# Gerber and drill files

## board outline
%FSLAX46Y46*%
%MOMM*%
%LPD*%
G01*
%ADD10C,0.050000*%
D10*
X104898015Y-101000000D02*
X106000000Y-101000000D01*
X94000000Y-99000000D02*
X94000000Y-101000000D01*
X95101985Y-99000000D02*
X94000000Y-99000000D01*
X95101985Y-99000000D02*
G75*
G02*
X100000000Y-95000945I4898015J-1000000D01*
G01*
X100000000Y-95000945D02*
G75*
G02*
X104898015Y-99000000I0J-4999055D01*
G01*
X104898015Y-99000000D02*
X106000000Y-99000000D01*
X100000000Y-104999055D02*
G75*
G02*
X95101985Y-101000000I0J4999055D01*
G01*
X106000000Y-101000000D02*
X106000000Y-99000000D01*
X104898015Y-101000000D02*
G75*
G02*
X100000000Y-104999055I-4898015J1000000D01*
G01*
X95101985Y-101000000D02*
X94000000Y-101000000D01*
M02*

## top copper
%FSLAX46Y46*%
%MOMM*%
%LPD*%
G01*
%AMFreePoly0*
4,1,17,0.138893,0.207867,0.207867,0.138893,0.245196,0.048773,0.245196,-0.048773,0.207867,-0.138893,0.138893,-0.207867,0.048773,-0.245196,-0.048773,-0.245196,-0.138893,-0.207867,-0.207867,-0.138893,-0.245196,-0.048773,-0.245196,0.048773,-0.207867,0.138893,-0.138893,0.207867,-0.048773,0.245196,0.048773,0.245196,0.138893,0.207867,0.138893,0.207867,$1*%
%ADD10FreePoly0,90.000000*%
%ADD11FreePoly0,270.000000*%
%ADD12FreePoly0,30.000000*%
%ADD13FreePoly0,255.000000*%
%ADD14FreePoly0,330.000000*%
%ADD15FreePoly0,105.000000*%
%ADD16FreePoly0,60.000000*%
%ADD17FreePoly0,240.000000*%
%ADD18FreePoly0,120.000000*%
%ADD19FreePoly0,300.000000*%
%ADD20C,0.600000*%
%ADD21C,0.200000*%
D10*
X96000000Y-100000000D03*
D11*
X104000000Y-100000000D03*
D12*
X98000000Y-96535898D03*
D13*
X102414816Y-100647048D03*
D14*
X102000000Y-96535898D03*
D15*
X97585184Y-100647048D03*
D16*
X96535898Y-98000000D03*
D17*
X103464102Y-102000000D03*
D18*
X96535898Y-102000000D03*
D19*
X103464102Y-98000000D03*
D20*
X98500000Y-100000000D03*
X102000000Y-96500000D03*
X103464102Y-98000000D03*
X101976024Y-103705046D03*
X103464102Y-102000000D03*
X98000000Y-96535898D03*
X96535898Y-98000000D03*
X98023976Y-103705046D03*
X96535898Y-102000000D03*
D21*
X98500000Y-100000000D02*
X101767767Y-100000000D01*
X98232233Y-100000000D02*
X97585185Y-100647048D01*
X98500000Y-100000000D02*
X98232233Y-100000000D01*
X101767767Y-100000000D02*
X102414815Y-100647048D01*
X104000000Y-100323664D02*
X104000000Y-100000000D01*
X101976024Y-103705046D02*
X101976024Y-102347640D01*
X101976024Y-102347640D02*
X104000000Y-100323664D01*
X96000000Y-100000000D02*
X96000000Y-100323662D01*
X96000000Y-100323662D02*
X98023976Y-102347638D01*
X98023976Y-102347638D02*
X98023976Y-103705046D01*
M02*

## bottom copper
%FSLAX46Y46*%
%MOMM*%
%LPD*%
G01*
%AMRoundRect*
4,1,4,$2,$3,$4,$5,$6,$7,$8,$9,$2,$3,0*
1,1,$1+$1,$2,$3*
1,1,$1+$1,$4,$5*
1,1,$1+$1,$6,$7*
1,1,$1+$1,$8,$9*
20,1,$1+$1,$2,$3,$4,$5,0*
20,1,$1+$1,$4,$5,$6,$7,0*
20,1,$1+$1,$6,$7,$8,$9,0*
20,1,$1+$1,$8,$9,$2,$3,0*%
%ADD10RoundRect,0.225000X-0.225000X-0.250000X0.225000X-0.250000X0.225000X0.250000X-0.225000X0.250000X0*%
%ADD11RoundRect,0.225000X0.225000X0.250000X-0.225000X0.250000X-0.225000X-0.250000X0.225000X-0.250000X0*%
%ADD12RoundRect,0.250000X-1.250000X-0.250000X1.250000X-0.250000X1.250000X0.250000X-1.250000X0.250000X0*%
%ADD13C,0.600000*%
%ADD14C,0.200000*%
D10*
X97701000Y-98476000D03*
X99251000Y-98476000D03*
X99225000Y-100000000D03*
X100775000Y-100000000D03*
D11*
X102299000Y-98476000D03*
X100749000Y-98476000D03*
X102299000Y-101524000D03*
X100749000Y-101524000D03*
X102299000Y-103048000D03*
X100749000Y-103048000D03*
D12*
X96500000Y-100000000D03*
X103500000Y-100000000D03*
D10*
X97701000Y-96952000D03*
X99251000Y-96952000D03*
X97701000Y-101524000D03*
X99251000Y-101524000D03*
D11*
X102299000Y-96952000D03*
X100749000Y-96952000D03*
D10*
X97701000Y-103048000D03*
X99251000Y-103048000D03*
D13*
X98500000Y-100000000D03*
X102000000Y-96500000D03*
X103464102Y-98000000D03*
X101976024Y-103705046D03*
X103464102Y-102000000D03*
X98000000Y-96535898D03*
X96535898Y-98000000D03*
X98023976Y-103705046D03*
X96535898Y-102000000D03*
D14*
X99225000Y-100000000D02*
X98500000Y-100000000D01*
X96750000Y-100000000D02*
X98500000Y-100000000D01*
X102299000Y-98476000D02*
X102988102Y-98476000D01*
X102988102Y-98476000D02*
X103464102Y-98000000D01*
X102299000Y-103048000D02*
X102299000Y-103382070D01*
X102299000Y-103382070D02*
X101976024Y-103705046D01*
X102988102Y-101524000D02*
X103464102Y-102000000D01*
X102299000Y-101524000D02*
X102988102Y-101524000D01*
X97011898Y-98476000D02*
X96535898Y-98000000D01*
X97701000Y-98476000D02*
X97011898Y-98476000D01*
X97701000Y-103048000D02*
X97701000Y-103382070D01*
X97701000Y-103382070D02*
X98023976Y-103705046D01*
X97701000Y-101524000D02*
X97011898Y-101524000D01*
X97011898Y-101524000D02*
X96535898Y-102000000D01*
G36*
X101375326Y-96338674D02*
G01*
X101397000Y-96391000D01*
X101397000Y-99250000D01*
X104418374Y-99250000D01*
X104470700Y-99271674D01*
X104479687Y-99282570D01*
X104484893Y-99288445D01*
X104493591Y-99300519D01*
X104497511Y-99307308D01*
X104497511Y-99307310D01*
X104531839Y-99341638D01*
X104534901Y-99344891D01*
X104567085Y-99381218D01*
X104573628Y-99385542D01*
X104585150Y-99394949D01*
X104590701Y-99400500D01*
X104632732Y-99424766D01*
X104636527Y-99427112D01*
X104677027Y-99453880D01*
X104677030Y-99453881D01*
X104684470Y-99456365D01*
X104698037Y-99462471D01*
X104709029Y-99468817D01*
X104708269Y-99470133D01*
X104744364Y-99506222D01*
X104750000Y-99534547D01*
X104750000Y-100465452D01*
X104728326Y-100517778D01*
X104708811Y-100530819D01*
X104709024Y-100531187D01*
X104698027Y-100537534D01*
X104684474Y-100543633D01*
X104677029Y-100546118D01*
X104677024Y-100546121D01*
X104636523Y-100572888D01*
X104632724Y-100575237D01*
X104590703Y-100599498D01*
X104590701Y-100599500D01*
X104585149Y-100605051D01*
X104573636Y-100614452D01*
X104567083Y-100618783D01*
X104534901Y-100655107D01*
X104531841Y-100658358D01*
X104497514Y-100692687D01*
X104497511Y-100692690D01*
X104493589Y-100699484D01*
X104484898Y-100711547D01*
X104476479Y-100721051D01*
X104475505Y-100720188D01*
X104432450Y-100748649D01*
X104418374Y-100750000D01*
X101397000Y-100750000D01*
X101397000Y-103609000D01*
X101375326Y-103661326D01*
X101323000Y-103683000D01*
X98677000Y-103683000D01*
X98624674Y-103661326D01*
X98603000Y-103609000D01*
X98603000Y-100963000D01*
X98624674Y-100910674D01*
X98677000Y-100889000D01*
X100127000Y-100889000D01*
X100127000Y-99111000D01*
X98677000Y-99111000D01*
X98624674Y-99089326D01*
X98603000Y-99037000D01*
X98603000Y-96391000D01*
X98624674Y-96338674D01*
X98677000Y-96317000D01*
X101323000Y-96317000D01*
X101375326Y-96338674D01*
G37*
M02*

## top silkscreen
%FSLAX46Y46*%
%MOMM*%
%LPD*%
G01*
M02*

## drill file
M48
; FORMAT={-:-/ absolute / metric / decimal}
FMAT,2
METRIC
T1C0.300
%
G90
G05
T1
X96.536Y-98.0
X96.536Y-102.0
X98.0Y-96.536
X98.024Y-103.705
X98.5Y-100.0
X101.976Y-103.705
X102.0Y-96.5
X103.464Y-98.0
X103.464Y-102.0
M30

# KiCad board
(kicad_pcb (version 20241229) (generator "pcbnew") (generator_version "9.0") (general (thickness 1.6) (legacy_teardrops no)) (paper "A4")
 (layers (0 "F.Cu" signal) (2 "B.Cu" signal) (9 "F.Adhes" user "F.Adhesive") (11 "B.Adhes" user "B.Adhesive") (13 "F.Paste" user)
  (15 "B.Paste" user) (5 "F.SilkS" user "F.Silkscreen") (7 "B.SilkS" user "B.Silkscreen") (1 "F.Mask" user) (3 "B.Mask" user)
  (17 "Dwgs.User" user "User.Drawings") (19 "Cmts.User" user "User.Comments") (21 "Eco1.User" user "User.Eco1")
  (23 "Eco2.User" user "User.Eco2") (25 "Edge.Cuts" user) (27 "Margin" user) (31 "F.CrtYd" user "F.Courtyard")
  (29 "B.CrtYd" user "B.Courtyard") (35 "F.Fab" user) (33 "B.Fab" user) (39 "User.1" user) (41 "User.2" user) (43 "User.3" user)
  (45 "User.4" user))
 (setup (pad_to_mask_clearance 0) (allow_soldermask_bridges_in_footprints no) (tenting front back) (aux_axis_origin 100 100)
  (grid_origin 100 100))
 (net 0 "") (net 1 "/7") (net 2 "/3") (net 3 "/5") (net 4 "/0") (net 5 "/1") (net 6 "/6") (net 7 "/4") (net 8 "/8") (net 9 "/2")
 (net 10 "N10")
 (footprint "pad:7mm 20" (layer "F.Cu") (at 100 100 90)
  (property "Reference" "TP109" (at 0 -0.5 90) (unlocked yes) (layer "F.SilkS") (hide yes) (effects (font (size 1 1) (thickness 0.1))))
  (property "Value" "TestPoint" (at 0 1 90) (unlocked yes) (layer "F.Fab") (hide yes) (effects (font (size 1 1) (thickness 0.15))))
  (pad "1" smd custom (at 0 -4 90) (size 0.5 0.5) (layers "F.Cu" "F.Mask" "F.Paste") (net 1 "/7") (thermal_bridge_angle 90)
   (options (clearance outline) (anchor circle)) (primitives)))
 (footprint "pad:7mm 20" (layer "F.Cu") (at 100 100 -90)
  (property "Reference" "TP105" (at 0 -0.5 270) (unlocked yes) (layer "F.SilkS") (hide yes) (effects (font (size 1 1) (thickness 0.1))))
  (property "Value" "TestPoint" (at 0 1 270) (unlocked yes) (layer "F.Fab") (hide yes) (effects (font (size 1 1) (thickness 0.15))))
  (pad "1" smd custom (at 0 -4 270) (size 0.5 0.5) (layers "F.Cu" "F.Mask" "F.Paste") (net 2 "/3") (thermal_bridge_angle 90)
   (options (clearance outline) (anchor circle)) (primitives)))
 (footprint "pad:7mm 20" (layer "F.Cu") (at 100 100 30)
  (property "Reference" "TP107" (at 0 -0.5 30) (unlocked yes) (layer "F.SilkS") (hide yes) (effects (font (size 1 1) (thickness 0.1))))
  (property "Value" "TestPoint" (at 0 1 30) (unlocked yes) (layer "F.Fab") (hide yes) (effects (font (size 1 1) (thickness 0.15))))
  (pad "1" smd custom (at 0 -4 30) (size 0.5 0.5) (layers "F.Cu" "F.Mask" "F.Paste") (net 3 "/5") (thermal_bridge_angle 90)
   (options (clearance outline) (anchor circle)) (primitives)))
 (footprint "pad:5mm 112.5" (layer "F.Cu") (at 100 100 -105)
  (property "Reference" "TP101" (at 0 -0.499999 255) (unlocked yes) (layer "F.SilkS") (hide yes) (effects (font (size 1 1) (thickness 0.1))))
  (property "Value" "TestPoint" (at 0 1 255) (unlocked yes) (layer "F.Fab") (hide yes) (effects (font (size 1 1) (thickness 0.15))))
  (pad "1" smd custom (at 0 -2.500001 255) (size 0.5 0.5) (layers "F.Cu" "F.Mask" "F.Paste") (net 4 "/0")
   (options (clearance outline) (anchor circle)) (primitives)))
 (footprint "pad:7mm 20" (layer "F.Cu") (at 100 100 -30)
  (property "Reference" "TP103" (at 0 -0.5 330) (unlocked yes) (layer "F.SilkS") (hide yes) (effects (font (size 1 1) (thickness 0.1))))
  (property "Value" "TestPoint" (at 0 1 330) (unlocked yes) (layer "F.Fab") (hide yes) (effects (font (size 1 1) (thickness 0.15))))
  (pad "1" smd custom (at 0 -4 330) (size 0.5 0.5) (layers "F.Cu" "F.Mask" "F.Paste") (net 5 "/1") (thermal_bridge_angle 90)
   (options (clearance outline) (anchor circle)) (primitives)))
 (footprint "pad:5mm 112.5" (layer "F.Cu") (at 100 100 105)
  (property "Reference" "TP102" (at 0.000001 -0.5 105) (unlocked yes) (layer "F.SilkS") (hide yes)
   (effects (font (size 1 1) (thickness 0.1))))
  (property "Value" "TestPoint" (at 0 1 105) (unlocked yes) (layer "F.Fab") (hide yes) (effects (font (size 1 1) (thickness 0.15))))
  (pad "1" smd custom (at 0 -2.500001 105) (size 0.5 0.5) (layers "F.Cu" "F.Mask" "F.Paste") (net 4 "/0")
   (options (clearance outline) (anchor circle)) (primitives)))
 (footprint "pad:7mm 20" (layer "F.Cu") (at 100 100 60)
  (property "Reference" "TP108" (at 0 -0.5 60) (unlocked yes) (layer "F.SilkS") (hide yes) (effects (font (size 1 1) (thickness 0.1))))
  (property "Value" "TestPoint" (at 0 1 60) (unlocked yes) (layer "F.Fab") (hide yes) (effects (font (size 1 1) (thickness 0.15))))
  (pad "1" smd custom (at 0 -4 60) (size 0.5 0.5) (layers "F.Cu" "F.Mask" "F.Paste") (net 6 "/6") (thermal_bridge_angle 90)
   (options (clearance outline) (anchor circle)) (primitives)))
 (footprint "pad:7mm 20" (layer "F.Cu") (at 100 100 -120)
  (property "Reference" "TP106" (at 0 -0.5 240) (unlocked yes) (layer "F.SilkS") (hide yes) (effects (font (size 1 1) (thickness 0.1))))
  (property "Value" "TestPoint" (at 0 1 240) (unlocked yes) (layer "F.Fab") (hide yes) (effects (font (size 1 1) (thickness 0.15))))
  (pad "1" smd custom (at 0 -4 240) (size 0.5 0.5) (layers "F.Cu" "F.Mask" "F.Paste") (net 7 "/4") (thermal_bridge_angle 90)
   (options (clearance outline) (anchor circle)) (primitives)))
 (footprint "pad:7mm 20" (layer "F.Cu") (at 100 100 120)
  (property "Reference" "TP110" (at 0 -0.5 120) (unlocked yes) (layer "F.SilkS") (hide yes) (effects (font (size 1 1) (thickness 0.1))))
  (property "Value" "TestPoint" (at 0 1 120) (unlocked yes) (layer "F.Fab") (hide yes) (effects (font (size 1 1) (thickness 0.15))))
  (pad "1" smd custom (at 0 -4 120) (size 0.5 0.5) (layers "F.Cu" "F.Mask" "F.Paste") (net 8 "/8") (thermal_bridge_angle 90)
   (options (clearance outline) (anchor circle)) (primitives)))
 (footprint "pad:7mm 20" (layer "F.Cu") (at 100 100 -60)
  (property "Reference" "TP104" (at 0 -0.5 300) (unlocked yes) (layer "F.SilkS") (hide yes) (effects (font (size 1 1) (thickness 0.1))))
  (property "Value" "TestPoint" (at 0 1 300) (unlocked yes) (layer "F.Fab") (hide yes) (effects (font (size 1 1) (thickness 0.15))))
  (pad "1" smd custom (at 0 -4 300) (size 0.5 0.5) (layers "F.Cu" "F.Mask" "F.Paste") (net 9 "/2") (thermal_bridge_angle 90)
   (options (clearance outline) (anchor circle)) (primitives)))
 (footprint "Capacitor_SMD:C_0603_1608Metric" (layer "B.Cu") (at 98.476 98.476)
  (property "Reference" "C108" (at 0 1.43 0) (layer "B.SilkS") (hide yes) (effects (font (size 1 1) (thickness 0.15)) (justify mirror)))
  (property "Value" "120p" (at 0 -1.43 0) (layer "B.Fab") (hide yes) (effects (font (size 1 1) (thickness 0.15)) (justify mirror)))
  (pad "1" smd roundrect (at -0.775 0) (size 0.9 0.95) (layers "B.Cu" "B.Mask" "B.Paste") (roundrect_rratio 0.25) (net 6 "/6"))
  (pad "2" smd roundrect (at 0.775 0) (size 0.9 0.95) (layers "B.Cu" "B.Mask" "B.Paste") (roundrect_rratio 0.25) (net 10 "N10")))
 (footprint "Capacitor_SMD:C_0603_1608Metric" (layer "B.Cu") (at 100 100)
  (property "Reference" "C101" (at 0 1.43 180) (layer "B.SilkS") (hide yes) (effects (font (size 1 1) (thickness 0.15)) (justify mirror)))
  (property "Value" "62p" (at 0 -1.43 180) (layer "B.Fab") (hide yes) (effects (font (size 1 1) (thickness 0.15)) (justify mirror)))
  (pad "1" smd roundrect (at -0.775 0) (size 0.9 0.95) (layers "B.Cu" "B.Mask" "B.Paste") (roundrect_rratio 0.25) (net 4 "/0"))
  (pad "2" smd roundrect (at 0.775 0) (size 0.9 0.95) (layers "B.Cu" "B.Mask" "B.Paste") (roundrect_rratio 0.25) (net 10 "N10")))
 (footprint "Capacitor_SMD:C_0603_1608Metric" (layer "B.Cu") (at 101.524 98.476 180)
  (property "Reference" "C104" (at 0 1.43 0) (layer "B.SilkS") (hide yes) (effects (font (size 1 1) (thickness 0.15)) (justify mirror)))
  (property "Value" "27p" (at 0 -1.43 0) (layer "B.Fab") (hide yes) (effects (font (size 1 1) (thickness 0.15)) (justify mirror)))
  (pad "1" smd roundrect (at -0.775 0 180) (size 0.9 0.95) (layers "B.Cu" "B.Mask" "B.Paste") (roundrect_rratio 0.25) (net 9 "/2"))
  (pad "2" smd roundrect (at 0.775 0 180) (size 0.9 0.95) (layers "B.Cu" "B.Mask" "B.Paste") (roundrect_rratio 0.25) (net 10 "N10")))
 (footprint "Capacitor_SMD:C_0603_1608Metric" (layer "B.Cu") (at 101.524 101.524 180)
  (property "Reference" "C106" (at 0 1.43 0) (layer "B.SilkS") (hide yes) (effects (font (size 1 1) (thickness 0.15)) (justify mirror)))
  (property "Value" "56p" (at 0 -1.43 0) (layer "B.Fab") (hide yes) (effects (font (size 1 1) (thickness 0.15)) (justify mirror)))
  (pad "1" smd roundrect (at -0.775 0 180) (size 0.9 0.95) (layers "B.Cu" "B.Mask" "B.Paste") (roundrect_rratio 0.25) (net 7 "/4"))
  (pad "2" smd roundrect (at 0.775 0 180) (size 0.9 0.95) (layers "B.Cu" "B.Mask" "B.Paste") (roundrect_rratio 0.25) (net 10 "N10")))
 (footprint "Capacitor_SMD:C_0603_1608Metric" (layer "B.Cu") (at 101.524 103.048 180)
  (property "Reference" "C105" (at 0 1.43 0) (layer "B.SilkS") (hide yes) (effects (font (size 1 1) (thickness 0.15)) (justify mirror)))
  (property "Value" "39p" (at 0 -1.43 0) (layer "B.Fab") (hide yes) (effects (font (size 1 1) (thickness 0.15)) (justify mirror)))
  (pad "1" smd roundrect (at -0.775 0 180) (size 0.9 0.95) (layers "B.Cu" "B.Mask" "B.Paste") (roundrect_rratio 0.25) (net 2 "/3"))
  (pad "2" smd roundrect (at 0.775 0 180) (size 0.9 0.95) (layers "B.Cu" "B.Mask" "B.Paste") (roundrect_rratio 0.25) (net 10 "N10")))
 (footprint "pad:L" (layer "B.Cu") (at 100 100)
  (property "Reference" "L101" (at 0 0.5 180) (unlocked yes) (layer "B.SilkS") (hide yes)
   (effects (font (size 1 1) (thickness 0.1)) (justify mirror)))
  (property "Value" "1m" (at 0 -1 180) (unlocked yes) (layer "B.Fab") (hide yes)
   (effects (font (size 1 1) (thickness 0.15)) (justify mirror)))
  (pad "1" smd roundrect (at -3.5 0) (size 3 1) (layers "B.Cu" "B.Mask" "B.Paste") (roundrect_rratio 0.25) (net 4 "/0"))
  (pad "2" smd roundrect (at 3.5 0) (size 3 1) (layers "B.Cu" "B.Mask" "B.Paste") (roundrect_rratio 0.25) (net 10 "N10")))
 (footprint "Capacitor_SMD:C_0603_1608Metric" (layer "B.Cu") (at 98.476 96.952)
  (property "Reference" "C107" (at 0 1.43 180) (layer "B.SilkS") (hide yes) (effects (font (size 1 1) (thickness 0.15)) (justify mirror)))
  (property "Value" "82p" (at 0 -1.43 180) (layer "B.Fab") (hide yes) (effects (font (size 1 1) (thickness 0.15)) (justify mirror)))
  (pad "1" smd roundrect (at -0.775 0) (size 0.9 0.95) (layers "B.Cu" "B.Mask" "B.Paste") (roundrect_rratio 0.25) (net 3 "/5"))
  (pad "2" smd roundrect (at 0.775 0) (size 0.9 0.95) (layers "B.Cu" "B.Mask" "B.Paste") (roundrect_rratio 0.25) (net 10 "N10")))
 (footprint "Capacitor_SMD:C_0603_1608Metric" (layer "B.Cu") (at 98.476 101.524)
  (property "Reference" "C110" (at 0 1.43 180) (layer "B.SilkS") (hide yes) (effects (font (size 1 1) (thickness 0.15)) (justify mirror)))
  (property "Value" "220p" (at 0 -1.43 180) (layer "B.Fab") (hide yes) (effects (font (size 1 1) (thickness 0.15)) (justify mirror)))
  (pad "1" smd roundrect (at -0.775 0) (size 0.9 0.95) (layers "B.Cu" "B.Mask" "B.Paste") (roundrect_rratio 0.25) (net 8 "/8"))
  (pad "2" smd roundrect (at 0.775 0) (size 0.9 0.95) (layers "B.Cu" "B.Mask" "B.Paste") (roundrect_rratio 0.25) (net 10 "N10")))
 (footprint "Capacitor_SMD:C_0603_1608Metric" (layer "B.Cu") (at 101.524 96.952 180)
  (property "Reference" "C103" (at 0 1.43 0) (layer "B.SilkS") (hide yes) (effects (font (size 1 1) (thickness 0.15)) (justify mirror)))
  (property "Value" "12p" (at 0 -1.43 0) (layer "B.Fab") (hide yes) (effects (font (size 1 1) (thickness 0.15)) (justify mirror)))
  (pad "1" smd roundrect (at -0.775 0 180) (size 0.9 0.95) (layers "B.Cu" "B.Mask" "B.Paste") (roundrect_rratio 0.25) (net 5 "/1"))
  (pad "2" smd roundrect (at 0.775 0 180) (size 0.9 0.95) (layers "B.Cu" "B.Mask" "B.Paste") (roundrect_rratio 0.25) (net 10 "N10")))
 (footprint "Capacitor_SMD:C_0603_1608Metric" (layer "B.Cu") (at 98.476 103.048)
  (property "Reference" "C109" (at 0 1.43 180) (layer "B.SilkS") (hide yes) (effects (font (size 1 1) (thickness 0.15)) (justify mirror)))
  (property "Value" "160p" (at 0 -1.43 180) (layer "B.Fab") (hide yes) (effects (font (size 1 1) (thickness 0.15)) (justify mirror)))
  (pad "1" smd roundrect (at -0.775 0) (size 0.9 0.95) (layers "B.Cu" "B.Mask" "B.Paste") (roundrect_rratio 0.25) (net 1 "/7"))
  (pad "2" smd roundrect (at 0.775 0) (size 0.9 0.95) (layers "B.Cu" "B.Mask" "B.Paste") (roundrect_rratio 0.25) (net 10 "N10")))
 (gr_line (start 104.898015 101) (end 106 101) (stroke (width 0.05) (type default)) (layer "Edge.Cuts"))
 (gr_line (start 94 99) (end 94 101) (stroke (width 0.05) (type default)) (layer "Edge.Cuts"))
 (gr_line (start 95.101985 99) (end 94 99) (stroke (width 0.05) (type default)) (layer "Edge.Cuts"))
 (gr_arc (start 95.101985 99) (mid 96.838395 96.127688) (end 100 95.000945) (stroke (width 0.05) (type default)) (layer "Edge.Cuts"))
 (gr_arc (start 100 95.000945) (mid 103.161605 96.127688) (end 104.898015 99) (stroke (width 0.05) (type default)) (layer "Edge.Cuts"))
 (gr_line (start 104.898015 99) (end 106 99) (stroke (width 0.05) (type default)) (layer "Edge.Cuts"))
 (gr_arc (start 100 104.999055) (mid 96.838395 103.872312) (end 95.101985 101) (stroke (width 0.05) (type default)) (layer "Edge.Cuts"))
 (gr_line (start 106 101) (end 106 99) (stroke (width 0.05) (type default)) (layer "Edge.Cuts"))
 (gr_arc (start 104.898015 101) (mid 103.161605 103.872312) (end 100 104.999055) (stroke (width 0.05) (type default)) (layer "Edge.Cuts"))
 (gr_line (start 95.101985 101) (end 94 101) (stroke (width 0.05) (type default)) (layer "Edge.Cuts"))
 (segment (start 98.5 100) (end 101.767767 100) (width 0.2) (layer "F.Cu") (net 4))
 (segment (start 98.232233 100) (end 97.585185 100.647048) (width 0.2) (layer "F.Cu") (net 4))
 (segment (start 98.5 100) (end 98.232233 100) (width 0.2) (layer "F.Cu") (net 4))
 (segment (start 101.767767 100) (end 102.414815 100.647048) (width 0.2) (layer "F.Cu") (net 4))
 (via (at 98.5 100) (size 0.6) (drill 0.3) (layers "F.Cu" "B.Cu") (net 4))
 (segment (start 99.225 100) (end 98.5 100) (width 0.2) (layer "B.Cu") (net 4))
 (segment (start 96.75 100) (end 98.5 100) (width 0.2) (layer "B.Cu") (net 4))
 (via (at 102 96.5) (size 0.6) (drill 0.3) (layers "F.Cu" "B.Cu") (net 5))
 (via (at 103.464102 98) (size 0.6) (drill 0.3) (layers "F.Cu" "B.Cu") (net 9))
 (segment (start 102.299 98.476) (end 102.988102 98.476) (width 0.2) (layer "B.Cu") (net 9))
 (segment (start 102.988102 98.476) (end 103.464102 98) (width 0.2) (layer "B.Cu") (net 9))
 (segment (start 104 100.323664) (end 104 100) (width 0.2) (layer "F.Cu") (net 2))
 (segment (start 101.976024 103.705046) (end 101.976024 102.34764) (width 0.2) (layer "F.Cu") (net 2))
 (segment (start 101.976024 102.34764) (end 104 100.323664) (width 0.2) (layer "F.Cu") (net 2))
 (via (at 101.976024 103.705046) (size 0.6) (drill 0.3) (layers "F.Cu" "B.Cu") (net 2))
 (segment (start 102.299 103.048) (end 102.299 103.38207) (width 0.2) (layer "B.Cu") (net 2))
 (segment (start 102.299 103.38207) (end 101.976024 103.705046) (width 0.2) (layer "B.Cu") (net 2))
 (via (at 103.464102 102) (size 0.6) (drill 0.3) (layers "F.Cu" "B.Cu") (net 7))
 (segment (start 102.988102 101.524) (end 103.464102 102) (width 0.2) (layer "B.Cu") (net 7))
 (segment (start 102.299 101.524) (end 102.988102 101.524) (width 0.2) (layer "B.Cu") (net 7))
 (via (at 98 96.535898) (size 0.6) (drill 0.3) (layers "F.Cu" "B.Cu") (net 3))
 (via (at 96.535898 98) (size 0.6) (drill 0.3) (layers "F.Cu" "B.Cu") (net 6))
 (segment (start 97.011898 98.476) (end 96.535898 98) (width 0.2) (layer "B.Cu") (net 6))
 (segment (start 97.701 98.476) (end 97.011898 98.476) (width 0.2) (layer "B.Cu") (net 6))
 (segment (start 96 100) (end 96 100.323662) (width 0.2) (layer "F.Cu") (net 1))
 (segment (start 96 100.323662) (end 98.023976 102.347638) (width 0.2) (layer "F.Cu") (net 1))
 (segment (start 98.023976 102.347638) (end 98.023976 103.705046) (width 0.2) (layer "F.Cu") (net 1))
 (via (at 98.023976 103.705046) (size 0.6) (drill 0.3) (layers "F.Cu" "B.Cu") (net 1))
 (segment (start 97.701 103.048) (end 97.701 103.38207) (width 0.2) (layer "B.Cu") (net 1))
 (segment (start 97.701 103.38207) (end 98.023976 103.705046) (width 0.2) (layer "B.Cu") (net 1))
 (via (at 96.535898 102) (size 0.6) (drill 0.3) (layers "F.Cu" "B.Cu") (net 8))
 (segment (start 97.701 101.524) (end 97.011898 101.524) (width 0.2) (layer "B.Cu") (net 8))
 (segment (start 97.011898 101.524) (end 96.535898 102) (width 0.2) (layer "B.Cu") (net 8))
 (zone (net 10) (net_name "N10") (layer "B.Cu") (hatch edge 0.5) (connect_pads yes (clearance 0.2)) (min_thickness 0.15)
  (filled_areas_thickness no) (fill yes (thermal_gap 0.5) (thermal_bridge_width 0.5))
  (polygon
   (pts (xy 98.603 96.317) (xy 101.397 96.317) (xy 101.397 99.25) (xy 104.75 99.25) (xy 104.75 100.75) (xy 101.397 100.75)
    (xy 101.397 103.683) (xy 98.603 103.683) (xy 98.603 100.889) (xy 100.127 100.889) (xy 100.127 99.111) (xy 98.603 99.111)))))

